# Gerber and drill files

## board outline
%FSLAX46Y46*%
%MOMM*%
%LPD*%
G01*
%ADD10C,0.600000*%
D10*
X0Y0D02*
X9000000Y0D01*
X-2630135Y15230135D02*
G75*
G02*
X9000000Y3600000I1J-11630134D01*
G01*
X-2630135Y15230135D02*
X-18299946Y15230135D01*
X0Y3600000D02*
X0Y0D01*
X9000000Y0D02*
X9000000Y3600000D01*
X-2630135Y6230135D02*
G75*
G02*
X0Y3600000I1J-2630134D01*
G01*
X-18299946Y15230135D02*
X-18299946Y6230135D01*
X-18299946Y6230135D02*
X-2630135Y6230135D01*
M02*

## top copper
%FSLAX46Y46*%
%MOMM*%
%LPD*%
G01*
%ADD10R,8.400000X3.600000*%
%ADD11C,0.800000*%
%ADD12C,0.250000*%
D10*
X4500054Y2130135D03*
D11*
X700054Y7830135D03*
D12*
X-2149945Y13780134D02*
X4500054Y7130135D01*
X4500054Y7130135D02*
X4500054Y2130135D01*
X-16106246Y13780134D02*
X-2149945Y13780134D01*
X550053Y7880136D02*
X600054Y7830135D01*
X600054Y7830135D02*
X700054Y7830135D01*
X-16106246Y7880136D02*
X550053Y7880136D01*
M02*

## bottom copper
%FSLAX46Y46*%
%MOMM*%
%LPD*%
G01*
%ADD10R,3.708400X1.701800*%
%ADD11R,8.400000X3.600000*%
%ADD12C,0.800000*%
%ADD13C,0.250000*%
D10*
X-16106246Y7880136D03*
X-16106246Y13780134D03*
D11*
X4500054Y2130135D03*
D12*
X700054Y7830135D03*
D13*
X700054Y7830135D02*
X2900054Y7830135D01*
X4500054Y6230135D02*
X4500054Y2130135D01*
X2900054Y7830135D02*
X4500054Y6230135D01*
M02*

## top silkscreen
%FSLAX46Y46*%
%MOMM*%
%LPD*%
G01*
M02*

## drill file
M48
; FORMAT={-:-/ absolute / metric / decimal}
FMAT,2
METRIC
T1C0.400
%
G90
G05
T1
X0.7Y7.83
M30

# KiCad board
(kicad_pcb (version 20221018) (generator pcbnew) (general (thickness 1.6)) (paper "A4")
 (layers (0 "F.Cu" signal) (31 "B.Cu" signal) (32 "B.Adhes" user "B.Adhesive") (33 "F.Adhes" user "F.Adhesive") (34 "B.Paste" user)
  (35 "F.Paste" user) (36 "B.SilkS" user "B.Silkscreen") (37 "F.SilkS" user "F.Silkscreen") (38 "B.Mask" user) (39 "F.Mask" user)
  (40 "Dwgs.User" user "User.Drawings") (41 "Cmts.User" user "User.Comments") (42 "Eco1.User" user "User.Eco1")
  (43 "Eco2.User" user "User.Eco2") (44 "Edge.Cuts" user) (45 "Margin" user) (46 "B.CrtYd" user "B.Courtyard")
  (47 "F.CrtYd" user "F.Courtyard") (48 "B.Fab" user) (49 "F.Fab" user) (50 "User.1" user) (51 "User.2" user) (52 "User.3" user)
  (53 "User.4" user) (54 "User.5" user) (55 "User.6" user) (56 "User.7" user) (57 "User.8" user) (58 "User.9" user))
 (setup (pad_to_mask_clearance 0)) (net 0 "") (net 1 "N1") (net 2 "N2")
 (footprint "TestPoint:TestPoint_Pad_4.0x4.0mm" (layer "F.Cu") (at 4.500054 -2.130135)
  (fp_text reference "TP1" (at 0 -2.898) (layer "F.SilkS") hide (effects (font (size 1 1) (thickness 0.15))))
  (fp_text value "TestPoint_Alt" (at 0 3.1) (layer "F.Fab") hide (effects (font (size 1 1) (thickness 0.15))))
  (pad "1" smd rect (at 0 0) (size 8.4 3.6) (layers "F.Cu" "F.Mask") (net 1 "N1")))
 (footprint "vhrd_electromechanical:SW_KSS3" (layer "B.Cu") (at -16.106246 -10.830135 90)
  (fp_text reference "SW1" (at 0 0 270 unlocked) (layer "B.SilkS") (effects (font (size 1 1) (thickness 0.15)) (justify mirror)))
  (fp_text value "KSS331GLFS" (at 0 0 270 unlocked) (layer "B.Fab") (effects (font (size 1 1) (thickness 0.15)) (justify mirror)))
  (pad "1" smd rect (at -2.949999 0 90) (size 1.7018 3.7084) (layers "B.Cu" "B.Paste" "B.Mask") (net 1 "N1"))
  (pad "2" smd rect (at 2.949999 0 90) (size 1.7018 3.7084) (layers "B.Cu" "B.Paste" "B.Mask") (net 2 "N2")))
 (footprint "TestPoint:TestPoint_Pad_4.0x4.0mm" (layer "B.Cu") (at 4.500054 -2.130135 180)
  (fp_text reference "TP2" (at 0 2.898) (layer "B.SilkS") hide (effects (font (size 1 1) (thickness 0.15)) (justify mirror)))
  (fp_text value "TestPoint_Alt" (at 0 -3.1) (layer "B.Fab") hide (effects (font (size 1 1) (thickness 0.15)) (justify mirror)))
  (pad "1" smd rect (at 0 0 180) (size 8.4 3.6) (layers "B.Cu" "B.Mask") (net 2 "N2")))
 (gr_line (start 0 0) (end 9 0) (stroke (width 0.6) (type solid)) (layer "Edge.Cuts"))
 (gr_arc (start -2.630135 -15.230135) (mid 5.593612 -11.823748) (end 9 -3.6) (stroke (width 0.6) (type solid)) (layer "Edge.Cuts"))
 (gr_line (start -2.630135 -15.230135) (end -18.299946 -15.230135) (stroke (width 0.6) (type solid)) (layer "Edge.Cuts"))
 (gr_line (start 0 -3.6) (end 0 0) (stroke (width 0.6) (type solid)) (layer "Edge.Cuts"))
 (gr_line (start 9 0) (end 9 -3.6) (stroke (width 0.6) (type solid)) (layer "Edge.Cuts"))
 (gr_arc (start -2.630135 -6.230135) (mid -0.770349 -5.459787) (end 0 -3.6) (stroke (width 0.6) (type solid)) (layer "Edge.Cuts"))
 (gr_line (start -18.299946 -15.230135) (end -18.299946 -6.230135) (stroke (width 0.6) (type solid)) (layer "Edge.Cuts"))
 (gr_line (start -18.299946 -6.230135) (end -2.630135 -6.230135) (stroke (width 0.6) (type solid)) (layer "Edge.Cuts"))
 (segment (start -2.149945 -13.780134) (end 4.500054 -7.130135) (width 0.25) (layer "F.Cu") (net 1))
 (segment (start 4.500054 -7.130135) (end 4.500054 -2.130135) (width 0.25) (layer "F.Cu") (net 1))
 (segment (start -16.106246 -13.780134) (end -2.149945 -13.780134) (width 0.25) (layer "F.Cu") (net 1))
 (segment (start 0.550053 -7.880136) (end 0.600054 -7.830135) (width 0.25) (layer "F.Cu") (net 2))
 (segment (start 0.600054 -7.830135) (end 0.700054 -7.830135) (width 0.25) (layer "F.Cu") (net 2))
 (segment (start -16.106246 -7.880136) (end 0.550053 -7.880136) (width 0.25) (layer "F.Cu") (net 2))
 (via (at 0.700054 -7.830135) (size 0.8) (drill 0.4) (layers "F.Cu" "B.Cu") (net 2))
 (segment (start 0.700054 -7.830135) (end 2.900054 -7.830135) (width 0.25) (layer "B.Cu") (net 2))
 (segment (start 4.500054 -6.230135) (end 4.500054 -2.130135) (width 0.25) (layer "B.Cu") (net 2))
 (segment (start 2.900054 -7.830135) (end 4.500054 -6.230135) (width 0.25) (layer "B.Cu") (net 2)))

